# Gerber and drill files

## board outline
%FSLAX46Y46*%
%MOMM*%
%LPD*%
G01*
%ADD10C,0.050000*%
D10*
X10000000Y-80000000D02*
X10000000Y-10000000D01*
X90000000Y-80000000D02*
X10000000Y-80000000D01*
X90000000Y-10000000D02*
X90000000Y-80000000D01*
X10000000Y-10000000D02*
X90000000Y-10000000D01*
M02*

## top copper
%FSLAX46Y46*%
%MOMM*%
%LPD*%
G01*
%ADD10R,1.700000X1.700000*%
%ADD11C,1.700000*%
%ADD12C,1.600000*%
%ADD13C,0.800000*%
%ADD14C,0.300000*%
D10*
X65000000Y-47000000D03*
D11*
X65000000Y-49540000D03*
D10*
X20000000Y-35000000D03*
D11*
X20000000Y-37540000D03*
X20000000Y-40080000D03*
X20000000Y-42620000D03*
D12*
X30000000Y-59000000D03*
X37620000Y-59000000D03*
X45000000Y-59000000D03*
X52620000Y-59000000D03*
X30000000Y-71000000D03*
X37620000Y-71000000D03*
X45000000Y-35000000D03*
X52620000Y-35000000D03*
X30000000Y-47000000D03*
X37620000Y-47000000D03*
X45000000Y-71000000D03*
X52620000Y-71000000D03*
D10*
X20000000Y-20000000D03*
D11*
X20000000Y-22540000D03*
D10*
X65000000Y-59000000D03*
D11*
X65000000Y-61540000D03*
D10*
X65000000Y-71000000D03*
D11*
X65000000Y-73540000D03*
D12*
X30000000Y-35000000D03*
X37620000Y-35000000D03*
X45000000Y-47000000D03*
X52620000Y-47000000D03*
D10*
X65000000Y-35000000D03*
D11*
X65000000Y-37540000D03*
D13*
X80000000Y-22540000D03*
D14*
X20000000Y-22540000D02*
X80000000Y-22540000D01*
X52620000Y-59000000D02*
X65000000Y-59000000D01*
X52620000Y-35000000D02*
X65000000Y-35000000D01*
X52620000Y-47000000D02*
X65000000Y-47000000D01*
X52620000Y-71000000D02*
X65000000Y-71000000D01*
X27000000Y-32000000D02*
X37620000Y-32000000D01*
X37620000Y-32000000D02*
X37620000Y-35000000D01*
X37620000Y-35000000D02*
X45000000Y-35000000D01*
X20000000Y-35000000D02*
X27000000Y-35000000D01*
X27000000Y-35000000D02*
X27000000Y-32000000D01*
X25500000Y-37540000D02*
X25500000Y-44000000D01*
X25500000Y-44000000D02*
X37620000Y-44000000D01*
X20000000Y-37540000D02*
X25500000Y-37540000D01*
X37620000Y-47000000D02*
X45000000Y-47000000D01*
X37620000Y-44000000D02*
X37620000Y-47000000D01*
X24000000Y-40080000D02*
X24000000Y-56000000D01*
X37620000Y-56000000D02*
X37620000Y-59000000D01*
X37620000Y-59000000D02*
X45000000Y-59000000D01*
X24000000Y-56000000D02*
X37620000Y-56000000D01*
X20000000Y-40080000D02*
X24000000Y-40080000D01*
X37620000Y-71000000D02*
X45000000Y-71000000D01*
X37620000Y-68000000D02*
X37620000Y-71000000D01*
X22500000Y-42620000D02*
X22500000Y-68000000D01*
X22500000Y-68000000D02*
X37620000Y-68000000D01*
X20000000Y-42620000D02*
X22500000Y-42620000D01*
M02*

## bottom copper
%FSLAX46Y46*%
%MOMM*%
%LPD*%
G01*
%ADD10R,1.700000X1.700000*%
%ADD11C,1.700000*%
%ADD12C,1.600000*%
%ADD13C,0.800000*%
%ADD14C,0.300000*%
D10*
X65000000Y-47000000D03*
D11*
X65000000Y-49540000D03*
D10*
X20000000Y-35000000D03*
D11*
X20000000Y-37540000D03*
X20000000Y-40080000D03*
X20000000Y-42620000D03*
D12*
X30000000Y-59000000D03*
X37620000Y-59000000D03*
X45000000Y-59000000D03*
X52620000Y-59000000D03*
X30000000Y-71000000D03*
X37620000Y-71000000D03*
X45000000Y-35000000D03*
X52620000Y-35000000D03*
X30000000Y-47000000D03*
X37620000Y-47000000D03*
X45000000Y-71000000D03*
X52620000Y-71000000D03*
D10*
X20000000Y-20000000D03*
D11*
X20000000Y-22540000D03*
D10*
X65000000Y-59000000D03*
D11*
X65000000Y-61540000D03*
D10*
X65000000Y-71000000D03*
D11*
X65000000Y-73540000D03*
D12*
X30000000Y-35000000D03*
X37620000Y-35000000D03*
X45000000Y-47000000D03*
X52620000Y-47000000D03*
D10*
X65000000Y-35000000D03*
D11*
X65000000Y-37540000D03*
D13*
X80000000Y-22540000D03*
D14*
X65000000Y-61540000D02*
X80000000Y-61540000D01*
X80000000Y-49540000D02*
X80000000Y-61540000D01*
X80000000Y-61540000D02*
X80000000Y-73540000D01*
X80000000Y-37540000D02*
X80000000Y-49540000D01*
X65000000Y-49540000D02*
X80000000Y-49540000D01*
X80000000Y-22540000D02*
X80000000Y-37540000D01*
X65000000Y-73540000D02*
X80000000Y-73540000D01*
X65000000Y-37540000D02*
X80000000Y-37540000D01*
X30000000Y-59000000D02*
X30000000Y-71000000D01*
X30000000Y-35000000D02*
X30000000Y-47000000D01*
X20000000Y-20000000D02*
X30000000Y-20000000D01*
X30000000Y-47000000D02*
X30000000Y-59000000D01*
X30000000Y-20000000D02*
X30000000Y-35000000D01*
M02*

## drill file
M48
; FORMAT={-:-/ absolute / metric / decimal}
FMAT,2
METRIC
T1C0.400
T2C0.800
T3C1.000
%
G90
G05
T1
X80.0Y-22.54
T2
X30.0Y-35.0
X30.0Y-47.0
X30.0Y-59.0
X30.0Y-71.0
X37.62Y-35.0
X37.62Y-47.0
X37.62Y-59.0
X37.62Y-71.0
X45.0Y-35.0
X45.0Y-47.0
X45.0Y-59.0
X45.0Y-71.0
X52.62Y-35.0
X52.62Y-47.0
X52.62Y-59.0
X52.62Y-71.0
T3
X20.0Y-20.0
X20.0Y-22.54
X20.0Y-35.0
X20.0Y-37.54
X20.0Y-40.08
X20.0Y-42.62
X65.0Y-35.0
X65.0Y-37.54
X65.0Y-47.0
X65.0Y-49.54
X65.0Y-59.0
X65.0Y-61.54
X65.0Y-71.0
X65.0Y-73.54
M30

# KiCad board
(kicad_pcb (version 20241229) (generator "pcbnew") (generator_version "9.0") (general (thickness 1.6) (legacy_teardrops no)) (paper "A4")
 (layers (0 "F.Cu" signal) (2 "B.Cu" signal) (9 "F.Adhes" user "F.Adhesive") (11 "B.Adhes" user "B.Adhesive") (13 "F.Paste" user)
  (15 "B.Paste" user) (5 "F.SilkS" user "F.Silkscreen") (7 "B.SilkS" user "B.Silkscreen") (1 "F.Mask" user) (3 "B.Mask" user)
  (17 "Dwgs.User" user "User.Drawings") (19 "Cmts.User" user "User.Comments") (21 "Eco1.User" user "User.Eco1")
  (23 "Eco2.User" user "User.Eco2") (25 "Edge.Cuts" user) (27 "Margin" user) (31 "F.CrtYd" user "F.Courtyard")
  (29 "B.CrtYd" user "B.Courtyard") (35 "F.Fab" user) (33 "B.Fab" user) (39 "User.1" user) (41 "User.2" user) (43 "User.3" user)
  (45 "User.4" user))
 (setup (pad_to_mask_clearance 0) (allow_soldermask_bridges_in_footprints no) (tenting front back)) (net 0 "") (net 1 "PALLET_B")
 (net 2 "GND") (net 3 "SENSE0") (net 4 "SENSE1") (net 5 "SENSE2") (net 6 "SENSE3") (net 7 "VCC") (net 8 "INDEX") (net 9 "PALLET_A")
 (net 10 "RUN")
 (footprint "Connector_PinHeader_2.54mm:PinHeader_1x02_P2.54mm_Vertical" (layer "F.Cu") (at 65 47)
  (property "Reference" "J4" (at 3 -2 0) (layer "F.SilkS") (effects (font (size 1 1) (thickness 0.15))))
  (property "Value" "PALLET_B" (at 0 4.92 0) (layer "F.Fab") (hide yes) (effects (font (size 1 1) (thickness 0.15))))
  (pad "1" thru_hole rect (at 0 0) (size 1.7 1.7) (drill 1) (layers "*.Cu" "*.Mask") (remove_unused_layers no) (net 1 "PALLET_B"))
  (pad "2" thru_hole circle (at 0 2.54) (size 1.7 1.7) (drill 1) (layers "*.Cu" "*.Mask") (remove_unused_layers no) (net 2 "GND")))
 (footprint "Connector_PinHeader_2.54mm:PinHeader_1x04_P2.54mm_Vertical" (layer "F.Cu") (at 20 35)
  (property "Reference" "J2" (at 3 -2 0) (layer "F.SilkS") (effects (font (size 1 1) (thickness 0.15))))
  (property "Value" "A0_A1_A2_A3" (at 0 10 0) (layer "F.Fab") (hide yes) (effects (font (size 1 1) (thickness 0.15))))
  (pad "1" thru_hole rect (at 0 0) (size 1.7 1.7) (drill 1) (layers "*.Cu" "*.Mask") (remove_unused_layers no) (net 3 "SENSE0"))
  (pad "2" thru_hole circle (at 0 2.54) (size 1.7 1.7) (drill 1) (layers "*.Cu" "*.Mask") (remove_unused_layers no) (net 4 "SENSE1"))
  (pad "3" thru_hole circle (at 0 5.08) (size 1.7 1.7) (drill 1) (layers "*.Cu" "*.Mask") (remove_unused_layers no) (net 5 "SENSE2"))
  (pad "4" thru_hole circle (at 0 7.62) (size 1.7 1.7) (drill 1) (layers "*.Cu" "*.Mask") (remove_unused_layers no) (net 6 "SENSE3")))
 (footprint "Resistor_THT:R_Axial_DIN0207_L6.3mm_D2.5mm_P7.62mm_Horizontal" (layer "F.Cu") (at 30 59)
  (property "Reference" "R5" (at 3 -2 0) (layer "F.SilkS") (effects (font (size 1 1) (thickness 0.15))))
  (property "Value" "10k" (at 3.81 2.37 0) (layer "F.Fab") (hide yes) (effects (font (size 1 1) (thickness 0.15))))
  (pad "1" thru_hole circle (at 0 0) (size 1.6 1.6) (drill 0.8) (layers "*.Cu" "*.Mask") (remove_unused_layers no) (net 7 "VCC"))
  (pad "2" thru_hole circle (at 7.62 0) (size 1.6 1.6) (drill 0.8) (layers "*.Cu" "*.Mask") (remove_unused_layers no) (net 5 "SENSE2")))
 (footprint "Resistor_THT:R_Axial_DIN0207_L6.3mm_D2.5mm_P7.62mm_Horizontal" (layer "F.Cu") (at 45 59)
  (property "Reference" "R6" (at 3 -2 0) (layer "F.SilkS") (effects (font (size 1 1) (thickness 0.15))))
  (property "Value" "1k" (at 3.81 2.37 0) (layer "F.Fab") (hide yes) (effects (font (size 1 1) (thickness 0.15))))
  (pad "1" thru_hole circle (at 0 0) (size 1.6 1.6) (drill 0.8) (layers "*.Cu" "*.Mask") (remove_unused_layers no) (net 5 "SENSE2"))
  (pad "2" thru_hole circle (at 7.62 0) (size 1.6 1.6) (drill 0.8) (layers "*.Cu" "*.Mask") (remove_unused_layers no) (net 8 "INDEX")))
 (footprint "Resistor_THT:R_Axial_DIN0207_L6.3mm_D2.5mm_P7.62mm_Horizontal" (layer "F.Cu") (at 30 71)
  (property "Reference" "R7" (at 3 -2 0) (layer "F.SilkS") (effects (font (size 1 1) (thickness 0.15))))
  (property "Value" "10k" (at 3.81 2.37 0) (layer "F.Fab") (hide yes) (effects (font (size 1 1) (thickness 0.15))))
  (pad "1" thru_hole circle (at 0 0) (size 1.6 1.6) (drill 0.8) (layers "*.Cu" "*.Mask") (remove_unused_layers no) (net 7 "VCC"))
  (pad "2" thru_hole circle (at 7.62 0) (size 1.6 1.6) (drill 0.8) (layers "*.Cu" "*.Mask") (remove_unused_layers no) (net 6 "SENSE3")))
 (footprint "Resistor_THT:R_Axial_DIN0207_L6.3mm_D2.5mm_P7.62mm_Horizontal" (layer "F.Cu") (at 45 35)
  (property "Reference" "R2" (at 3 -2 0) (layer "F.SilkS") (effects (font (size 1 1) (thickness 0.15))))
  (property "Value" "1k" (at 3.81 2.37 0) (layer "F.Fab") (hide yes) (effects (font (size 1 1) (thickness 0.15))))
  (pad "1" thru_hole circle (at 0 0) (size 1.6 1.6) (drill 0.8) (layers "*.Cu" "*.Mask") (remove_unused_layers no) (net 3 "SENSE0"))
  (pad "2" thru_hole circle (at 7.62 0) (size 1.6 1.6) (drill 0.8) (layers "*.Cu" "*.Mask") (remove_unused_layers no) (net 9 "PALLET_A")))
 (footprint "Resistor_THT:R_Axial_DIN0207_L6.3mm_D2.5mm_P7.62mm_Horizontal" (layer "F.Cu") (at 30 47)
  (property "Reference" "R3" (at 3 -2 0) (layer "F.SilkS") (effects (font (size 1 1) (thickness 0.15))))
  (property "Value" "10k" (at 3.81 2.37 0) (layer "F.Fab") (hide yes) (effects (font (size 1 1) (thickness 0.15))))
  (pad "1" thru_hole circle (at 0 0) (size 1.6 1.6) (drill 0.8) (layers "*.Cu" "*.Mask") (remove_unused_layers no) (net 7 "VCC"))
  (pad "2" thru_hole circle (at 7.62 0) (size 1.6 1.6) (drill 0.8) (layers "*.Cu" "*.Mask") (remove_unused_layers no) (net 4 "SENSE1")))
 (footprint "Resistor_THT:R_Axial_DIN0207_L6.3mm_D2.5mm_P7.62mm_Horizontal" (layer "F.Cu") (at 45 71)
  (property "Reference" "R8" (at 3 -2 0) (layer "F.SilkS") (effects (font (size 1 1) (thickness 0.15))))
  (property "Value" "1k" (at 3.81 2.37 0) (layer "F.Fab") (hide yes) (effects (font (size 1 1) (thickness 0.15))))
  (pad "1" thru_hole circle (at 0 0) (size 1.6 1.6) (drill 0.8) (layers "*.Cu" "*.Mask") (remove_unused_layers no) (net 6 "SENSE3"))
  (pad "2" thru_hole circle (at 7.62 0) (size 1.6 1.6) (drill 0.8) (layers "*.Cu" "*.Mask") (remove_unused_layers no) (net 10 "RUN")))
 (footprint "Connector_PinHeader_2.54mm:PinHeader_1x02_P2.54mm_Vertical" (layer "F.Cu") (at 20 20)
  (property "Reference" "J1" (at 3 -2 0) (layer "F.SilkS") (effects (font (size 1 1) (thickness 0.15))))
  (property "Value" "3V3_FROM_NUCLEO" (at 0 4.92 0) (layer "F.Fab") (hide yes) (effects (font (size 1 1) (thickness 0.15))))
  (pad "1" thru_hole rect (at 0 0) (size 1.7 1.7) (drill 1) (layers "*.Cu" "*.Mask") (remove_unused_layers no) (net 7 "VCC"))
  (pad "2" thru_hole circle (at 0 2.54) (size 1.7 1.7) (drill 1) (layers "*.Cu" "*.Mask") (remove_unused_layers no) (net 2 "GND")))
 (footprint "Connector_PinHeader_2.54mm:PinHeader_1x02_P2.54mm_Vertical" (layer "F.Cu") (at 65 59)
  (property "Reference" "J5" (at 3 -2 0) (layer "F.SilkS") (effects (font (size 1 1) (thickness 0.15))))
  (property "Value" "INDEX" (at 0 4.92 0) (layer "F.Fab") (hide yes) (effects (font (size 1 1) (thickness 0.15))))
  (pad "1" thru_hole rect (at 0 0) (size 1.7 1.7) (drill 1) (layers "*.Cu" "*.Mask") (remove_unused_layers no) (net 8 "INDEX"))
  (pad "2" thru_hole circle (at 0 2.54) (size 1.7 1.7) (drill 1) (layers "*.Cu" "*.Mask") (remove_unused_layers no) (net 2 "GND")))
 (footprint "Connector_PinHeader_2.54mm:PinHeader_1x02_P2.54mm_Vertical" (layer "F.Cu") (at 65 71)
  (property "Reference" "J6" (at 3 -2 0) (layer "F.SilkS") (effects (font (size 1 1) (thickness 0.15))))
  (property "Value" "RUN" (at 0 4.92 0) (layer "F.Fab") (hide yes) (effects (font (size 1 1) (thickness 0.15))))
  (pad "1" thru_hole rect (at 0 0) (size 1.7 1.7) (drill 1) (layers "*.Cu" "*.Mask") (remove_unused_layers no) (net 10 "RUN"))
  (pad "2" thru_hole circle (at 0 2.54) (size 1.7 1.7) (drill 1) (layers "*.Cu" "*.Mask") (remove_unused_layers no) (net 2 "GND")))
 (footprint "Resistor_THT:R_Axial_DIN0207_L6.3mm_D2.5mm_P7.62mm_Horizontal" (layer "F.Cu") (at 30 35)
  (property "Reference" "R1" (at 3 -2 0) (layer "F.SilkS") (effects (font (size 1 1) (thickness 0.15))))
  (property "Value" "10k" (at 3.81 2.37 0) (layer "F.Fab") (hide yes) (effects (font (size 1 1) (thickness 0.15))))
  (pad "1" thru_hole circle (at 0 0) (size 1.6 1.6) (drill 0.8) (layers "*.Cu" "*.Mask") (remove_unused_layers no) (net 7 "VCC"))
  (pad "2" thru_hole circle (at 7.62 0) (size 1.6 1.6) (drill 0.8) (layers "*.Cu" "*.Mask") (remove_unused_layers no) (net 3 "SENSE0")))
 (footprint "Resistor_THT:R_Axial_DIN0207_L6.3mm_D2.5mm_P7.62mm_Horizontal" (layer "F.Cu") (at 45 47)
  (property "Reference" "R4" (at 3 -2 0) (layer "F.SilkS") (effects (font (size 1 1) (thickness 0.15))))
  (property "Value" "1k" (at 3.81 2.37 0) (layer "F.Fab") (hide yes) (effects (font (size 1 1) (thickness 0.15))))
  (pad "1" thru_hole circle (at 0 0) (size 1.6 1.6) (drill 0.8) (layers "*.Cu" "*.Mask") (remove_unused_layers no) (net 4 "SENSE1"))
  (pad "2" thru_hole circle (at 7.62 0) (size 1.6 1.6) (drill 0.8) (layers "*.Cu" "*.Mask") (remove_unused_layers no) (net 1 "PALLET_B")))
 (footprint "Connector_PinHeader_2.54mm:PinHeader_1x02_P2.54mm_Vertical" (layer "F.Cu") (at 65 35)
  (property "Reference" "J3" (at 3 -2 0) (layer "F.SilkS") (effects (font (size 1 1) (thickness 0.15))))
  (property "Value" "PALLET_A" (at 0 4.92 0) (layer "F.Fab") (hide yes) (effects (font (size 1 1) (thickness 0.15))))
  (pad "1" thru_hole rect (at 0 0) (size 1.7 1.7) (drill 1) (layers "*.Cu" "*.Mask") (remove_unused_layers no) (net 9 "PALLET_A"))
  (pad "2" thru_hole circle (at 0 2.54) (size 1.7 1.7) (drill 1) (layers "*.Cu" "*.Mask") (remove_unused_layers no) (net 2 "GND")))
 (gr_line (start 10 80) (end 10 10) (stroke (width 0.05) (type default)) (layer "Edge.Cuts"))
 (gr_line (start 90 80) (end 10 80) (stroke (width 0.05) (type default)) (layer "Edge.Cuts"))
 (gr_line (start 90 10) (end 90 80) (stroke (width 0.05) (type default)) (layer "Edge.Cuts"))
 (gr_line (start 10 10) (end 90 10) (stroke (width 0.05) (type default)) (layer "Edge.Cuts"))
 (segment (start 20 22.54) (end 80 22.54) (width 0.3) (layer "F.Cu") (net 2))
 (via (at 80 22.54) (size 0.8) (drill 0.4) (layers "F.Cu" "B.Cu") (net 2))
 (segment (start 65 61.54) (end 80 61.54) (width 0.3) (layer "B.Cu") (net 2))
 (segment (start 80 49.54) (end 80 61.54) (width 0.3) (layer "B.Cu") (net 2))
 (segment (start 80 61.54) (end 80 73.54) (width 0.3) (layer "B.Cu") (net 2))
 (segment (start 80 37.54) (end 80 49.54) (width 0.3) (layer "B.Cu") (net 2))
 (segment (start 65 49.54) (end 80 49.54) (width 0.3) (layer "B.Cu") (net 2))
 (segment (start 80 22.54) (end 80 37.54) (width 0.3) (layer "B.Cu") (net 2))
 (segment (start 65 73.54) (end 80 73.54) (width 0.3) (layer "B.Cu") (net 2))
 (segment (start 65 37.54) (end 80 37.54) (width 0.3) (layer "B.Cu") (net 2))
 (segment (start 52.62 59) (end 65 59) (width 0.3) (layer "F.Cu") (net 8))
 (segment (start 52.62 35) (end 65 35) (width 0.3) (layer "F.Cu") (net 9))
 (segment (start 52.62 47) (end 65 47) (width 0.3) (layer "F.Cu") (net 1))
 (segment (start 52.62 71) (end 65 71) (width 0.3) (layer "F.Cu") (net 10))
 (segment (start 27 32) (end 37.62 32) (width 0.3) (layer "F.Cu") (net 3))
 (segment (start 37.62 32) (end 37.62 35) (width 0.3) (layer "F.Cu") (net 3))
 (segment (start 37.62 35) (end 45 35) (width 0.3) (layer "F.Cu") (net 3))
 (segment (start 20 35) (end 27 35) (width 0.3) (layer "F.Cu") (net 3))
 (segment (start 27 35) (end 27 32) (width 0.3) (layer "F.Cu") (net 3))
 (segment (start 25.5 37.54) (end 25.5 44) (width 0.3) (layer "F.Cu") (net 4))
 (segment (start 25.5 44) (end 37.62 44) (width 0.3) (layer "F.Cu") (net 4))
 (segment (start 20 37.54) (end 25.5 37.54) (width 0.3) (layer "F.Cu") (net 4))
 (segment (start 37.62 47) (end 45 47) (width 0.3) (layer "F.Cu") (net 4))
 (segment (start 37.62 44) (end 37.62 47) (width 0.3) (layer "F.Cu") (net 4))
 (segment (start 24 40.08) (end 24 56) (width 0.3) (layer "F.Cu") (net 5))
 (segment (start 37.62 56) (end 37.62 59) (width 0.3) (layer "F.Cu") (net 5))
 (segment (start 37.62 59) (end 45 59) (width 0.3) (layer "F.Cu") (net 5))
 (segment (start 24 56) (end 37.62 56) (width 0.3) (layer "F.Cu") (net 5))
 (segment (start 20 40.08) (end 24 40.08) (width 0.3) (layer "F.Cu") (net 5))
 (segment (start 37.62 71) (end 45 71) (width 0.3) (layer "F.Cu") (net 6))
 (segment (start 37.62 68) (end 37.62 71) (width 0.3) (layer "F.Cu") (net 6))
 (segment (start 22.5 42.62) (end 22.5 68) (width 0.3) (layer "F.Cu") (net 6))
 (segment (start 22.5 68) (end 37.62 68) (width 0.3) (layer "F.Cu") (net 6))
 (segment (start 20 42.62) (end 22.5 42.62) (width 0.3) (layer "F.Cu") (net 6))
 (segment (start 30 59) (end 30 71) (width 0.3) (layer "B.Cu") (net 7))
 (segment (start 30 35) (end 30 47) (width 0.3) (layer "B.Cu") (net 7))
 (segment (start 20 20) (end 30 20) (width 0.3) (layer "B.Cu") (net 7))
 (segment (start 30 47) (end 30 59) (width 0.3) (layer "B.Cu") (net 7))
 (segment (start 30 20) (end 30 35) (width 0.3) (layer "B.Cu") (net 7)))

